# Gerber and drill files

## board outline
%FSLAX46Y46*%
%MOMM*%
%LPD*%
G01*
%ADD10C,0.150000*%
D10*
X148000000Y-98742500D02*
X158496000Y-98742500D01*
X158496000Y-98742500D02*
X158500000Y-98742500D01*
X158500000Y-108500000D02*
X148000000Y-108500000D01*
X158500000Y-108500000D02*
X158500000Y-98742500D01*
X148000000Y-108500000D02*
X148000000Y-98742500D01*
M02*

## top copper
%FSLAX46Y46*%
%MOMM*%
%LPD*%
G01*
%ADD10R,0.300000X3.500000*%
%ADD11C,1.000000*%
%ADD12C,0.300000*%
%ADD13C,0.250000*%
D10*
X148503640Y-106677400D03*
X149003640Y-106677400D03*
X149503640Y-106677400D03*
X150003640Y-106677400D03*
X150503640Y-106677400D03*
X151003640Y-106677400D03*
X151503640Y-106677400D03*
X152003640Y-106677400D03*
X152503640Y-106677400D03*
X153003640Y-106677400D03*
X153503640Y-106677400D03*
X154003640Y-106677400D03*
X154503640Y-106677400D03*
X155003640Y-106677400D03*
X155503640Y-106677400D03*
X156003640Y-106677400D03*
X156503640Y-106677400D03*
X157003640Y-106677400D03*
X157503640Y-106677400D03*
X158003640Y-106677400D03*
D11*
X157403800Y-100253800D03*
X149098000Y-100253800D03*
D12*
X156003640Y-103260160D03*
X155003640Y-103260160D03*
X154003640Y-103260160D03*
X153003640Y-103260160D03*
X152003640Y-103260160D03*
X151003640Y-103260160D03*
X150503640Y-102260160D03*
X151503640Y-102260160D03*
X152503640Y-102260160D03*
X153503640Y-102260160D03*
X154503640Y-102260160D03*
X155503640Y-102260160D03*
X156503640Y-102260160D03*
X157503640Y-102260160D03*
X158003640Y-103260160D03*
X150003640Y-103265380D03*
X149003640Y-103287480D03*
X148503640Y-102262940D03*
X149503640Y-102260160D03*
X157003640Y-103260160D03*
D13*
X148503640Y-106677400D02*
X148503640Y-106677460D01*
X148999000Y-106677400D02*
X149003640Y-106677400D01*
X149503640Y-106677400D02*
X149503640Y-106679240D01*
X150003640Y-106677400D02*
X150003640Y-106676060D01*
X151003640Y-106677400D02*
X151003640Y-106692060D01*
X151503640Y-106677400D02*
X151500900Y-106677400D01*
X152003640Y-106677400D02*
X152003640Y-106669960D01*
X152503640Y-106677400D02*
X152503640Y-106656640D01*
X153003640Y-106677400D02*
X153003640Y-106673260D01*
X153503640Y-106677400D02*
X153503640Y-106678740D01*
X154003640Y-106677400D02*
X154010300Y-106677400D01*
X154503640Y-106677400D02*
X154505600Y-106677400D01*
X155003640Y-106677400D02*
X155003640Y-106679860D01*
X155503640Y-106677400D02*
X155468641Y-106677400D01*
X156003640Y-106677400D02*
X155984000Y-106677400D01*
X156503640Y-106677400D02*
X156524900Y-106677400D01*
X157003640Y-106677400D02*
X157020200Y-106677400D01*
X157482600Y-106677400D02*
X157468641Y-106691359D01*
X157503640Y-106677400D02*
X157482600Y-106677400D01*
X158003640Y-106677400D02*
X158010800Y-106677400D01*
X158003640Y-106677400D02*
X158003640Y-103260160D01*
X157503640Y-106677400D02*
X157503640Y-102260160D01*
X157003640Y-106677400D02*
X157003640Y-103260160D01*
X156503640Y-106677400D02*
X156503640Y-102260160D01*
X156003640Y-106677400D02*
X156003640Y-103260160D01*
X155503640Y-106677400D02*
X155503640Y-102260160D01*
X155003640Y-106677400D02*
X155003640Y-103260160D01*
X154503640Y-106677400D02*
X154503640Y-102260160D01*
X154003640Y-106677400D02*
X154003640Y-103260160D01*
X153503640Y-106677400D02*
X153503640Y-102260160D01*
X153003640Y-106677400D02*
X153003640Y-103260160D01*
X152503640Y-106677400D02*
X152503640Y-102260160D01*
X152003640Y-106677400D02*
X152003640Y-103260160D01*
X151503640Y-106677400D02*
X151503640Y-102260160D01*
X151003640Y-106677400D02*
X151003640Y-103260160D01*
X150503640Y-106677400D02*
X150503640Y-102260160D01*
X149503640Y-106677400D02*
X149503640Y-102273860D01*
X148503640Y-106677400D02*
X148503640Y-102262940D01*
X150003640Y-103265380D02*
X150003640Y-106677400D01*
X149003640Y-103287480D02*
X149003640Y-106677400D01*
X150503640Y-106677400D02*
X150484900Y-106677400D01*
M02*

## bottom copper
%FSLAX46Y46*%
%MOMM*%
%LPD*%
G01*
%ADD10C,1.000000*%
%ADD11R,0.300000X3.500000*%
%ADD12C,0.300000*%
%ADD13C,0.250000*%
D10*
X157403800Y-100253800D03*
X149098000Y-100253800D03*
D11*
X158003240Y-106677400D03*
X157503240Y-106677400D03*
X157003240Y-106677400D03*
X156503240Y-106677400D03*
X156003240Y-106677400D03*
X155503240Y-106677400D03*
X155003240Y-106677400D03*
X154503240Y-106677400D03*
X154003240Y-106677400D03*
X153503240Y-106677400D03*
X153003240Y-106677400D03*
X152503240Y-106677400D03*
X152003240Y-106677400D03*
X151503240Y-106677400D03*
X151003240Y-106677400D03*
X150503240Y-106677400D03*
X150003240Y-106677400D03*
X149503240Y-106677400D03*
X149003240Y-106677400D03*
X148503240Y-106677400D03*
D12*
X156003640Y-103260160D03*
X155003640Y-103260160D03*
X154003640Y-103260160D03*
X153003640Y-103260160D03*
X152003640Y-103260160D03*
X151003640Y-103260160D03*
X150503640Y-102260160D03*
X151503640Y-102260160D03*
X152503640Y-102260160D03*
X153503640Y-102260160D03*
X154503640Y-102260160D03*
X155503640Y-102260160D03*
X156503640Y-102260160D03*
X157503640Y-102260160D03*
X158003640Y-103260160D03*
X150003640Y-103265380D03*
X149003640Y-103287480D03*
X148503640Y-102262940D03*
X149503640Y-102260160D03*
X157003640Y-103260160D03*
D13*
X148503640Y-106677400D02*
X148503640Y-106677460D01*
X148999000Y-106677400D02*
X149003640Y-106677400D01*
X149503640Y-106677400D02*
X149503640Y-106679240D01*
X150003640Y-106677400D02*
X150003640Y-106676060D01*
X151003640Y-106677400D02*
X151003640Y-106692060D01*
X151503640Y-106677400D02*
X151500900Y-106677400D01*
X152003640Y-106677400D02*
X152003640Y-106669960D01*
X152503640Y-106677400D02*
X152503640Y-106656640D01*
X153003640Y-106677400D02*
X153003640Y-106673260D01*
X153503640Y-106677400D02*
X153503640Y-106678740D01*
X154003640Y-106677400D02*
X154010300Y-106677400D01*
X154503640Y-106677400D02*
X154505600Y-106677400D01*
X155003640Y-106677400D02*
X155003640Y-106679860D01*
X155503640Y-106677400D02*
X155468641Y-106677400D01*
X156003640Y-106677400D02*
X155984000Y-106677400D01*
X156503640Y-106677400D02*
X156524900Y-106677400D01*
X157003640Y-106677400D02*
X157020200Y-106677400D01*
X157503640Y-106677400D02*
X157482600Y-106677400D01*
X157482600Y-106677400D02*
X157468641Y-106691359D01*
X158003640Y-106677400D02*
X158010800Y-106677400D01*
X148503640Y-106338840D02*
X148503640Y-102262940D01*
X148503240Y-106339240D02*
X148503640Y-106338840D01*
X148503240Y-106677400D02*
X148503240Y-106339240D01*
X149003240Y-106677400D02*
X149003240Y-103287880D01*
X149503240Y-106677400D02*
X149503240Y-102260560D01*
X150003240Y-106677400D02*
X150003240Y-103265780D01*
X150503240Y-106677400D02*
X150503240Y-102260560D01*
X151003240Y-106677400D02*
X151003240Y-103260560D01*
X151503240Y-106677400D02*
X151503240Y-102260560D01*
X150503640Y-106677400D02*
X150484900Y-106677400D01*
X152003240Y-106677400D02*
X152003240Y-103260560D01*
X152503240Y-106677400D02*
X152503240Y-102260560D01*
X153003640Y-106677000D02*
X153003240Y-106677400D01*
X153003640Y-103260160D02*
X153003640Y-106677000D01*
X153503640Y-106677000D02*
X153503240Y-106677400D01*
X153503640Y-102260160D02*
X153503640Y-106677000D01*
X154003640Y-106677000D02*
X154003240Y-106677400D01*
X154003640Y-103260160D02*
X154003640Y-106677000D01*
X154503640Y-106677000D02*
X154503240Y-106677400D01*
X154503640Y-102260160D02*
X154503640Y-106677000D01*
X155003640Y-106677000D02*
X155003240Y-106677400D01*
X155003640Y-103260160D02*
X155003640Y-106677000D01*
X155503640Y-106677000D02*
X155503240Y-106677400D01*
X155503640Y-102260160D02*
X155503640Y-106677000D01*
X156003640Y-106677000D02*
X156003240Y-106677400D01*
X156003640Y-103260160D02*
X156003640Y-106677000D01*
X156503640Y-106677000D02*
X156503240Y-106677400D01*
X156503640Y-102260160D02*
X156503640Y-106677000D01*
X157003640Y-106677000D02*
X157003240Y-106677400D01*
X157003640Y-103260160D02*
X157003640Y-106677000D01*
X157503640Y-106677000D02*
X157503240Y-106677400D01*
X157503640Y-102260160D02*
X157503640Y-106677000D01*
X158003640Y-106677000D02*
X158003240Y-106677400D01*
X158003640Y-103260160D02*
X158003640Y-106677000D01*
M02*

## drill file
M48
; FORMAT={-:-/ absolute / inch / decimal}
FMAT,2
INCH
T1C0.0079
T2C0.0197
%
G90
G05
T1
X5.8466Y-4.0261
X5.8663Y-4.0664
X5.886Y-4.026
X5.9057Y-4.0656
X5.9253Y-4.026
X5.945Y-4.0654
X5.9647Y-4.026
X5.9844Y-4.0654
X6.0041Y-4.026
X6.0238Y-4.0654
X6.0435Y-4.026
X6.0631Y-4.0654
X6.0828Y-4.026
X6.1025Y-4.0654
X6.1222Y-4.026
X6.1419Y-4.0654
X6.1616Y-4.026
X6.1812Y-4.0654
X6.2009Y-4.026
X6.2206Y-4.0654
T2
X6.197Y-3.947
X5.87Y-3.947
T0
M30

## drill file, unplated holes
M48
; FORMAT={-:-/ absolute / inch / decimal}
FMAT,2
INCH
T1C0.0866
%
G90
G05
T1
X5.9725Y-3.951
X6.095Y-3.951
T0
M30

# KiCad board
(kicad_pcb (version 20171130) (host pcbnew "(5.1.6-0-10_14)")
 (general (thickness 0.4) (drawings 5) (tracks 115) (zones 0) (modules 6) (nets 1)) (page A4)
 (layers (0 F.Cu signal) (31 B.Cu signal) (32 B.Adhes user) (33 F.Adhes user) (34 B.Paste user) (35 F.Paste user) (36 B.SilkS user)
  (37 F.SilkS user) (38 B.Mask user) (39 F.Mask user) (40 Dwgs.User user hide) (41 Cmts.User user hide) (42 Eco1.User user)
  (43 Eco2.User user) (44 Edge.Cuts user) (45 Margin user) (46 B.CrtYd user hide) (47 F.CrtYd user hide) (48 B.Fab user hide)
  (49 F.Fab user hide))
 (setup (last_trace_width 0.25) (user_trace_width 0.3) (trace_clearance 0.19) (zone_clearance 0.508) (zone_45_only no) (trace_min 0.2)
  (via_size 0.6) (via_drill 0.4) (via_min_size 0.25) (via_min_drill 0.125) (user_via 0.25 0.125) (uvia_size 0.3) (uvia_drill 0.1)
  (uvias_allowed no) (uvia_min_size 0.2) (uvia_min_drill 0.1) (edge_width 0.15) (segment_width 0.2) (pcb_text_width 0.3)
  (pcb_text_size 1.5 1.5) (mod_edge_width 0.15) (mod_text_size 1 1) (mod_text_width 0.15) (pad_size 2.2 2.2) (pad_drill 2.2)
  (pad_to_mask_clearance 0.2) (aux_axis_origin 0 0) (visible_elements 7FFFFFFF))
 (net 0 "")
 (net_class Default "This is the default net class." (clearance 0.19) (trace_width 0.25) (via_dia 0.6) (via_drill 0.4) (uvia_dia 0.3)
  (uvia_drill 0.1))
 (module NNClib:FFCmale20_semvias (layer F.Cu) (at 148.50364 104.9274)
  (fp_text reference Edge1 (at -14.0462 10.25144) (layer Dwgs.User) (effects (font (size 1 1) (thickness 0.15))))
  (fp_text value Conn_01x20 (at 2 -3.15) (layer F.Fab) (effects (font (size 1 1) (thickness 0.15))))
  (pad 1 smd rect (at 0 1.75) (size 0.3 3.5) (layers *.Paste *.Mask F.Cu))
  (pad 2 smd rect (at 0.5 1.75) (size 0.3 3.5) (layers *.Paste *.Mask F.Cu))
  (pad 3 smd rect (at 1 1.75) (size 0.3 3.5) (layers *.Paste *.Mask F.Cu))
  (pad 4 smd rect (at 1.5 1.75) (size 0.3 3.5) (layers *.Paste *.Mask F.Cu))
  (pad 5 smd rect (at 2 1.75) (size 0.3 3.5) (layers *.Paste *.Mask F.Cu))
  (pad 6 smd rect (at 2.5 1.75) (size 0.3 3.5) (layers *.Paste *.Mask F.Cu))
  (pad 7 smd rect (at 3 1.75) (size 0.3 3.5) (layers *.Paste *.Mask F.Cu))
  (pad 8 smd rect (at 3.5 1.75) (size 0.3 3.5) (layers *.Paste *.Mask F.Cu))
  (pad 9 smd rect (at 4 1.75) (size 0.3 3.5) (layers *.Paste *.Mask F.Cu))
  (pad 10 smd rect (at 4.5 1.75) (size 0.3 3.5) (layers *.Paste *.Mask F.Cu))
  (pad 11 smd rect (at 5 1.75) (size 0.3 3.5) (layers *.Paste *.Mask F.Cu))
  (pad 12 smd rect (at 5.5 1.75) (size 0.3 3.5) (layers *.Paste *.Mask F.Cu))
  (pad 13 smd rect (at 6 1.75) (size 0.3 3.5) (layers *.Paste *.Mask F.Cu))
  (pad 14 smd rect (at 6.5 1.75) (size 0.3 3.5) (layers *.Paste *.Mask F.Cu))
  (pad 15 smd rect (at 7 1.75) (size 0.3 3.5) (layers *.Paste *.Mask F.Cu))
  (pad 16 smd rect (at 7.5 1.75) (size 0.3 3.5) (layers *.Paste *.Mask F.Cu))
  (pad 17 smd rect (at 8 1.75) (size 0.3 3.5) (layers *.Paste *.Mask F.Cu))
  (pad 18 smd rect (at 8.5 1.75) (size 0.3 3.5) (layers *.Paste *.Mask F.Cu))
  (pad 19 smd rect (at 9 1.75) (size 0.3 3.5) (layers *.Paste *.Mask F.Cu))
  (pad 20 smd rect (at 9.5 1.75) (size 0.3 3.5) (layers *.Paste *.Mask F.Cu)))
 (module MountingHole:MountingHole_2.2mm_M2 (layer F.Cu) (at 151.7015 100.3554)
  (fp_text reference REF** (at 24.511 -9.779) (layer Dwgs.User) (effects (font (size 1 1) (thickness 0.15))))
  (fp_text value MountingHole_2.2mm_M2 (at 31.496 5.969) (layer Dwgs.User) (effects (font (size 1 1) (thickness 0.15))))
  (pad 1 np_thru_hole circle (at 0 0) (size 2.2 2.2) (drill 2.2) (layers *.Cu *.Mask)))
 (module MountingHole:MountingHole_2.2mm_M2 (layer F.Cu) (at 154.813 100.3554)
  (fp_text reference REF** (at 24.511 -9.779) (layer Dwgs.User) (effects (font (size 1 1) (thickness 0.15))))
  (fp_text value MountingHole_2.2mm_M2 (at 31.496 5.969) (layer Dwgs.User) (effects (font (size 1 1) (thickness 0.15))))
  (pad 1 np_thru_hole circle (at 0 0) (size 2.2 2.2) (drill 2.2) (layers *.Cu *.Mask)))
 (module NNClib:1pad (layer F.Cu) (at 157.4038 100.2538)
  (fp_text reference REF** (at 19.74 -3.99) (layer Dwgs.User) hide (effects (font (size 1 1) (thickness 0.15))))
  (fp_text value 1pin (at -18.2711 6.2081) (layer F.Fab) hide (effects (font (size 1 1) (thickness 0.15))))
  (pad 1 thru_hole circle (at 0 0) (size 1 1) (drill 0.5) (layers *.Cu *.Mask)))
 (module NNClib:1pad (layer F.Cu) (at 149.098 100.2538)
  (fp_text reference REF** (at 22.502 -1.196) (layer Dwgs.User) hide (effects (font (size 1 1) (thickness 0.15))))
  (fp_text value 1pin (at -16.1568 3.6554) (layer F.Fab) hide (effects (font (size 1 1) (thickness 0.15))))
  (pad 1 thru_hole circle (at 0 0) (size 1 1) (drill 0.5) (layers *.Cu *.Mask)))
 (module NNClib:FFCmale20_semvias (layer B.Cu) (at 158.00324 104.9274 180)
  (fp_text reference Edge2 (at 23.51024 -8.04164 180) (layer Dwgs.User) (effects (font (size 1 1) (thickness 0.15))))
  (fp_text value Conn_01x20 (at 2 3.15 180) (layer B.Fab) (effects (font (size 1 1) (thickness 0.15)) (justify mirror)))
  (pad 1 smd rect (at 0 -1.75 180) (size 0.3 3.5) (layers *.Paste *.Mask B.Cu))
  (pad 2 smd rect (at 0.5 -1.75 180) (size 0.3 3.5) (layers *.Paste *.Mask B.Cu))
  (pad 3 smd rect (at 1 -1.75 180) (size 0.3 3.5) (layers *.Paste *.Mask B.Cu))
  (pad 4 smd rect (at 1.5 -1.75 180) (size 0.3 3.5) (layers *.Paste *.Mask B.Cu))
  (pad 5 smd rect (at 2 -1.75 180) (size 0.3 3.5) (layers *.Paste *.Mask B.Cu))
  (pad 6 smd rect (at 2.5 -1.75 180) (size 0.3 3.5) (layers *.Paste *.Mask B.Cu))
  (pad 7 smd rect (at 3 -1.75 180) (size 0.3 3.5) (layers *.Paste *.Mask B.Cu))
  (pad 8 smd rect (at 3.5 -1.75 180) (size 0.3 3.5) (layers *.Paste *.Mask B.Cu))
  (pad 9 smd rect (at 4 -1.75 180) (size 0.3 3.5) (layers *.Paste *.Mask B.Cu))
  (pad 10 smd rect (at 4.5 -1.75 180) (size 0.3 3.5) (layers *.Paste *.Mask B.Cu))
  (pad 11 smd rect (at 5 -1.75 180) (size 0.3 3.5) (layers *.Paste *.Mask B.Cu))
  (pad 12 smd rect (at 5.5 -1.75 180) (size 0.3 3.5) (layers *.Paste *.Mask B.Cu))
  (pad 13 smd rect (at 6 -1.75 180) (size 0.3 3.5) (layers *.Paste *.Mask B.Cu))
  (pad 14 smd rect (at 6.5 -1.75 180) (size 0.3 3.5) (layers *.Paste *.Mask B.Cu))
  (pad 15 smd rect (at 7 -1.75 180) (size 0.3 3.5) (layers *.Paste *.Mask B.Cu))
  (pad 16 smd rect (at 7.5 -1.75 180) (size 0.3 3.5) (layers *.Paste *.Mask B.Cu))
  (pad 17 smd rect (at 8 -1.75 180) (size 0.3 3.5) (layers *.Paste *.Mask B.Cu))
  (pad 18 smd rect (at 8.5 -1.75 180) (size 0.3 3.5) (layers *.Paste *.Mask B.Cu))
  (pad 19 smd rect (at 9 -1.75 180) (size 0.3 3.5) (layers *.Paste *.Mask B.Cu))
  (pad 20 smd rect (at 9.5 -1.75 180) (size 0.3 3.5) (layers *.Paste *.Mask B.Cu)))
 (gr_line (start 148 98.7425) (end 158.496 98.7425) (layer Edge.Cuts) (width 0.15))
 (gr_line (start 158.496 98.7425) (end 158.5 98.7425) (layer Edge.Cuts) (width 0.15))
 (gr_line (start 158.5 108.5) (end 148 108.5) (angle 90) (layer Edge.Cuts) (width 0.15))
 (gr_line (start 158.5 108.5) (end 158.5 98.7425) (angle 90) (layer Edge.Cuts) (width 0.15))
 (gr_line (start 148 108.5) (end 148 98.7425) (angle 90) (layer Edge.Cuts) (width 0.15))
 (segment (start 148.50364 106.6774) (end 148.50364 106.67746) (width 0.25) (layer B.Cu) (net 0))
 (segment (start 148.999 106.6774) (end 149.00364 106.6774) (width 0.25) (layer B.Cu) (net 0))
 (segment (start 149.50364 106.6774) (end 149.50364 106.67924) (width 0.25) (layer B.Cu) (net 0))
 (segment (start 150.00364 106.6774) (end 150.00364 106.67606) (width 0.25) (layer B.Cu) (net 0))
 (segment (start 151.00364 106.6774) (end 151.00364 106.69206) (width 0.25) (layer B.Cu) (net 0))
 (segment (start 151.50364 106.6774) (end 151.5009 106.6774) (width 0.25) (layer B.Cu) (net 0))
 (segment (start 152.00364 106.6774) (end 152.00364 106.66996) (width 0.25) (layer B.Cu) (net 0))
 (segment (start 152.50364 106.6774) (end 152.50364 106.65664) (width 0.25) (layer B.Cu) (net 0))
 (segment (start 153.00364 106.6774) (end 153.00364 106.67326) (width 0.25) (layer B.Cu) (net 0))
 (segment (start 153.50364 106.6774) (end 153.50364 106.67874) (width 0.25) (layer B.Cu) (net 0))
 (segment (start 154.00364 106.6774) (end 154.0103 106.6774) (width 0.25) (layer B.Cu) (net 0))
 (segment (start 154.50364 106.6774) (end 154.5056 106.6774) (width 0.25) (layer B.Cu) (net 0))
 (segment (start 155.00364 106.6774) (end 155.00364 106.67986) (width 0.25) (layer B.Cu) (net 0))
 (segment (start 155.50364 106.6774) (end 155.468641 106.6774) (width 0.25) (layer B.Cu) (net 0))
 (segment (start 156.00364 106.6774) (end 155.984 106.6774) (width 0.25) (layer B.Cu) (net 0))
 (segment (start 156.50364 106.6774) (end 156.5249 106.6774) (width 0.25) (layer B.Cu) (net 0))
 (segment (start 157.00364 106.6774) (end 157.0202 106.6774) (width 0.25) (layer B.Cu) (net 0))
 (segment (start 157.50364 106.6774) (end 157.4826 106.6774) (width 0.25) (layer B.Cu) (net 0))
 (segment (start 157.4826 106.6774) (end 157.468641 106.691359) (width 0.25) (layer B.Cu) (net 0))
 (segment (start 158.00364 106.6774) (end 158.0108 106.6774) (width 0.25) (layer B.Cu) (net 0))
 (segment (start 148.50364 106.6774) (end 148.50364 106.67746) (width 0.25) (layer F.Cu) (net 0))
 (segment (start 148.999 106.6774) (end 149.00364 106.6774) (width 0.25) (layer F.Cu) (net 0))
 (segment (start 149.50364 106.6774) (end 149.50364 106.67924) (width 0.25) (layer F.Cu) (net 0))
 (segment (start 150.00364 106.6774) (end 150.00364 106.67606) (width 0.25) (layer F.Cu) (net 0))
 (segment (start 151.00364 106.6774) (end 151.00364 106.69206) (width 0.25) (layer F.Cu) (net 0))
 (segment (start 151.50364 106.6774) (end 151.5009 106.6774) (width 0.25) (layer F.Cu) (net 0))
 (segment (start 152.00364 106.6774) (end 152.00364 106.66996) (width 0.25) (layer F.Cu) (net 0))
 (segment (start 152.50364 106.6774) (end 152.50364 106.65664) (width 0.25) (layer F.Cu) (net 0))
 (segment (start 153.00364 106.6774) (end 153.00364 106.67326) (width 0.25) (layer F.Cu) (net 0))
 (segment (start 153.50364 106.6774) (end 153.50364 106.67874) (width 0.25) (layer F.Cu) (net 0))
 (segment (start 154.00364 106.6774) (end 154.0103 106.6774) (width 0.25) (layer F.Cu) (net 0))
 (segment (start 154.50364 106.6774) (end 154.5056 106.6774) (width 0.25) (layer F.Cu) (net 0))
 (segment (start 155.00364 106.6774) (end 155.00364 106.67986) (width 0.25) (layer F.Cu) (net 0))
 (segment (start 155.50364 106.6774) (end 155.468641 106.6774) (width 0.25) (layer F.Cu) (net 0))
 (segment (start 156.00364 106.6774) (end 155.984 106.6774) (width 0.25) (layer F.Cu) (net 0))
 (segment (start 156.50364 106.6774) (end 156.5249 106.6774) (width 0.25) (layer F.Cu) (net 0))
 (segment (start 157.00364 106.6774) (end 157.0202 106.6774) (width 0.25) (layer F.Cu) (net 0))
 (segment (start 157.4826 106.6774) (end 157.468641 106.691359) (width 0.25) (layer F.Cu) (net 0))
 (segment (start 157.50364 106.6774) (end 157.4826 106.6774) (width 0.25) (layer F.Cu) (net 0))
 (segment (start 158.00364 106.6774) (end 158.0108 106.6774) (width 0.25) (layer F.Cu) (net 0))
 (segment (start 158.00364 106.6774) (end 158.00364 103.26016) (width 0.25) (layer F.Cu) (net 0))
 (segment (start 157.50364 106.6774) (end 157.50364 102.26016) (width 0.25) (layer F.Cu) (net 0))
 (segment (start 157.00364 106.6774) (end 157.00364 103.26016) (width 0.25) (layer F.Cu) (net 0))
 (segment (start 156.50364 106.6774) (end 156.50364 102.26016) (width 0.25) (layer F.Cu) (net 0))
 (segment (start 156.00364 106.6774) (end 156.00364 103.26016) (width 0.25) (layer F.Cu) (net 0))
 (segment (start 155.50364 106.6774) (end 155.50364 102.26016) (width 0.25) (layer F.Cu) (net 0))
 (segment (start 155.00364 106.6774) (end 155.00364 103.26016) (width 0.25) (layer F.Cu) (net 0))
 (segment (start 154.50364 106.6774) (end 154.50364 102.26016) (width 0.25) (layer F.Cu) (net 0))
 (segment (start 154.00364 106.6774) (end 154.00364 103.26016) (width 0.25) (layer F.Cu) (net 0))
 (segment (start 153.50364 106.6774) (end 153.50364 102.26016) (width 0.25) (layer F.Cu) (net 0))
 (segment (start 153.00364 106.6774) (end 153.00364 103.26016) (width 0.25) (layer F.Cu) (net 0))
 (segment (start 152.50364 106.6774) (end 152.50364 102.26016) (width 0.25) (layer F.Cu) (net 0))
 (segment (start 152.00364 106.6774) (end 152.00364 103.26016) (width 0.25) (layer F.Cu) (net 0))
 (segment (start 151.50364 106.6774) (end 151.50364 102.26016) (width 0.25) (layer F.Cu) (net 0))
 (segment (start 151.00364 106.6774) (end 151.00364 103.26016) (width 0.25) (layer F.Cu) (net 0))
 (segment (start 150.50364 106.6774) (end 150.50364 102.26016) (width 0.25) (layer F.Cu) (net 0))
 (segment (start 149.50364 106.6774) (end 149.50364 102.27386) (width 0.25) (layer F.Cu) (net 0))
 (via (at 156.00364 103.26016) (size 0.3) (drill 0.2) (layers F.Cu B.Cu) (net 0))
 (via (at 155.00364 103.26016) (size 0.3) (drill 0.2) (layers F.Cu B.Cu) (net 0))
 (via (at 154.00364 103.26016) (size 0.3) (drill 0.2) (layers F.Cu B.Cu) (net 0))
 (via (at 153.00364 103.26016) (size 0.3) (drill 0.2) (layers F.Cu B.Cu) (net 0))
 (via (at 152.00364 103.26016) (size 0.3) (drill 0.2) (layers F.Cu B.Cu) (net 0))
 (via (at 151.00364 103.26016) (size 0.3) (drill 0.2) (layers F.Cu B.Cu) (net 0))
 (via (at 150.50364 102.26016) (size 0.3) (drill 0.2) (layers F.Cu B.Cu) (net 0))
 (via (at 151.50364 102.26016) (size 0.3) (drill 0.2) (layers F.Cu B.Cu) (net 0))
 (via (at 152.50364 102.26016) (size 0.3) (drill 0.2) (layers F.Cu B.Cu) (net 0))
 (via (at 153.50364 102.26016) (size 0.3) (drill 0.2) (layers F.Cu B.Cu) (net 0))
 (via (at 154.50364 102.26016) (size 0.3) (drill 0.2) (layers F.Cu B.Cu) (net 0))
 (via (at 155.50364 102.26016) (size 0.3) (drill 0.2) (layers F.Cu B.Cu) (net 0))
 (via (at 156.50364 102.26016) (size 0.3) (drill 0.2) (layers F.Cu B.Cu) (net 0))
 (via (at 157.50364 102.26016) (size 0.3) (drill 0.2) (layers F.Cu B.Cu) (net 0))
 (via (at 158.00364 103.26016) (size 0.3) (drill 0.2) (layers F.Cu B.Cu) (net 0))
 (segment (start 148.50364 106.6774) (end 148.50364 102.26294) (width 0.25) (layer F.Cu) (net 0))
 (segment (start 150.00364 103.26538) (end 150.00364 106.6774) (width 0.25) (layer F.Cu) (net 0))
 (via (at 150.00364 103.26538) (size 0.3) (drill 0.2) (layers F.Cu B.Cu) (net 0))
 (segment (start 149.00364 103.28748) (end 149.00364 106.6774) (width 0.25) (layer F.Cu) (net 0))
 (via (at 149.00364 103.28748) (size 0.3) (drill 0.2) (layers F.Cu B.Cu) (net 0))
 (via (at 148.50364 102.26294) (size 0.3) (drill 0.2) (layers F.Cu B.Cu) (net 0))
 (via (at 149.50364 102.26016) (size 0.3) (drill 0.2) (layers F.Cu B.Cu) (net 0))
 (segment (start 148.50364 106.33884) (end 148.50364 102.26294) (width 0.25) (layer B.Cu) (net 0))
 (segment (start 148.50324 106.33924) (end 148.50364 106.33884) (width 0.25) (layer B.Cu) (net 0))
 (segment (start 148.50324 106.6774) (end 148.50324 106.33924) (width 0.25) (layer B.Cu) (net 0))
 (segment (start 149.00324 106.6774) (end 149.00324 103.28788) (width 0.25) (layer B.Cu) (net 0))
 (segment (start 149.50324 106.6774) (end 149.50324 102.26056) (width 0.25) (layer B.Cu) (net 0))
 (segment (start 150.00324 106.6774) (end 150.00324 103.26578) (width 0.25) (layer B.Cu) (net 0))
 (segment (start 150.50324 106.6774) (end 150.50324 102.26056) (width 0.25) (layer B.Cu) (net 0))
 (segment (start 151.00324 106.6774) (end 151.00324 103.26056) (width 0.25) (layer B.Cu) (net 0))
 (segment (start 151.50324 106.6774) (end 151.50324 102.26056) (width 0.25) (layer B.Cu) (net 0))
 (segment (start 150.50364 106.6774) (end 150.4849 106.6774) (width 0.25) (layer F.Cu) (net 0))
 (segment (start 150.50364 106.6774) (end 150.4849 106.6774) (width 0.25) (layer B.Cu) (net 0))
 (segment (start 152.00324 106.6774) (end 152.00324 103.26056) (width 0.25) (layer B.Cu) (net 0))
 (segment (start 152.50324 106.6774) (end 152.50324 102.26056) (width 0.25) (layer B.Cu) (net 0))
 (segment (start 153.00364 106.677) (end 153.00324 106.6774) (width 0.25) (layer B.Cu) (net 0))
 (segment (start 153.00364 103.26016) (end 153.00364 106.677) (width 0.25) (layer B.Cu) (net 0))
 (segment (start 153.50364 106.677) (end 153.50324 106.6774) (width 0.25) (layer B.Cu) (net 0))
 (segment (start 153.50364 102.26016) (end 153.50364 106.677) (width 0.25) (layer B.Cu) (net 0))
 (segment (start 154.00364 106.677) (end 154.00324 106.6774) (width 0.25) (layer B.Cu) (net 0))
 (segment (start 154.00364 103.26016) (end 154.00364 106.677) (width 0.25) (layer B.Cu) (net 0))
 (segment (start 154.50364 106.677) (end 154.50324 106.6774) (width 0.25) (layer B.Cu) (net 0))
 (segment (start 154.50364 102.26016) (end 154.50364 106.677) (width 0.25) (layer B.Cu) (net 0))
 (segment (start 155.00364 106.677) (end 155.00324 106.6774) (width 0.25) (layer B.Cu) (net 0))
 (segment (start 155.00364 103.26016) (end 155.00364 106.677) (width 0.25) (layer B.Cu) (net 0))
 (segment (start 155.50364 106.677) (end 155.50324 106.6774) (width 0.25) (layer B.Cu) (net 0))
 (segment (start 155.50364 102.26016) (end 155.50364 106.677) (width 0.25) (layer B.Cu) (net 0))
 (segment (start 156.00364 106.677) (end 156.00324 106.6774) (width 0.25) (layer B.Cu) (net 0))
 (segment (start 156.00364 103.26016) (end 156.00364 106.677) (width 0.25) (layer B.Cu) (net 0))
 (segment (start 156.50364 106.677) (end 156.50324 106.6774) (width 0.25) (layer B.Cu) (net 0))
 (segment (start 156.50364 102.26016) (end 156.50364 106.677) (width 0.25) (layer B.Cu) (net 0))
 (segment (start 157.00364 106.677) (end 157.00324 106.6774) (width 0.25) (layer B.Cu) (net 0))
 (segment (start 157.00364 103.26016) (end 157.00364 106.677) (width 0.25) (layer B.Cu) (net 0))
 (segment (start 157.50364 106.677) (end 157.50324 106.6774) (width 0.25) (layer B.Cu) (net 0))
 (segment (start 157.50364 102.26016) (end 157.50364 106.677) (width 0.25) (layer B.Cu) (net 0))
 (segment (start 158.00364 106.677) (end 158.00324 106.6774) (width 0.25) (layer B.Cu) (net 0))
 (segment (start 158.00364 103.26016) (end 158.00364 106.677) (width 0.25) (layer B.Cu) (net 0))
 (via (at 157.00364 103.26016) (size 0.3) (drill 0.2) (layers F.Cu B.Cu) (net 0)))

